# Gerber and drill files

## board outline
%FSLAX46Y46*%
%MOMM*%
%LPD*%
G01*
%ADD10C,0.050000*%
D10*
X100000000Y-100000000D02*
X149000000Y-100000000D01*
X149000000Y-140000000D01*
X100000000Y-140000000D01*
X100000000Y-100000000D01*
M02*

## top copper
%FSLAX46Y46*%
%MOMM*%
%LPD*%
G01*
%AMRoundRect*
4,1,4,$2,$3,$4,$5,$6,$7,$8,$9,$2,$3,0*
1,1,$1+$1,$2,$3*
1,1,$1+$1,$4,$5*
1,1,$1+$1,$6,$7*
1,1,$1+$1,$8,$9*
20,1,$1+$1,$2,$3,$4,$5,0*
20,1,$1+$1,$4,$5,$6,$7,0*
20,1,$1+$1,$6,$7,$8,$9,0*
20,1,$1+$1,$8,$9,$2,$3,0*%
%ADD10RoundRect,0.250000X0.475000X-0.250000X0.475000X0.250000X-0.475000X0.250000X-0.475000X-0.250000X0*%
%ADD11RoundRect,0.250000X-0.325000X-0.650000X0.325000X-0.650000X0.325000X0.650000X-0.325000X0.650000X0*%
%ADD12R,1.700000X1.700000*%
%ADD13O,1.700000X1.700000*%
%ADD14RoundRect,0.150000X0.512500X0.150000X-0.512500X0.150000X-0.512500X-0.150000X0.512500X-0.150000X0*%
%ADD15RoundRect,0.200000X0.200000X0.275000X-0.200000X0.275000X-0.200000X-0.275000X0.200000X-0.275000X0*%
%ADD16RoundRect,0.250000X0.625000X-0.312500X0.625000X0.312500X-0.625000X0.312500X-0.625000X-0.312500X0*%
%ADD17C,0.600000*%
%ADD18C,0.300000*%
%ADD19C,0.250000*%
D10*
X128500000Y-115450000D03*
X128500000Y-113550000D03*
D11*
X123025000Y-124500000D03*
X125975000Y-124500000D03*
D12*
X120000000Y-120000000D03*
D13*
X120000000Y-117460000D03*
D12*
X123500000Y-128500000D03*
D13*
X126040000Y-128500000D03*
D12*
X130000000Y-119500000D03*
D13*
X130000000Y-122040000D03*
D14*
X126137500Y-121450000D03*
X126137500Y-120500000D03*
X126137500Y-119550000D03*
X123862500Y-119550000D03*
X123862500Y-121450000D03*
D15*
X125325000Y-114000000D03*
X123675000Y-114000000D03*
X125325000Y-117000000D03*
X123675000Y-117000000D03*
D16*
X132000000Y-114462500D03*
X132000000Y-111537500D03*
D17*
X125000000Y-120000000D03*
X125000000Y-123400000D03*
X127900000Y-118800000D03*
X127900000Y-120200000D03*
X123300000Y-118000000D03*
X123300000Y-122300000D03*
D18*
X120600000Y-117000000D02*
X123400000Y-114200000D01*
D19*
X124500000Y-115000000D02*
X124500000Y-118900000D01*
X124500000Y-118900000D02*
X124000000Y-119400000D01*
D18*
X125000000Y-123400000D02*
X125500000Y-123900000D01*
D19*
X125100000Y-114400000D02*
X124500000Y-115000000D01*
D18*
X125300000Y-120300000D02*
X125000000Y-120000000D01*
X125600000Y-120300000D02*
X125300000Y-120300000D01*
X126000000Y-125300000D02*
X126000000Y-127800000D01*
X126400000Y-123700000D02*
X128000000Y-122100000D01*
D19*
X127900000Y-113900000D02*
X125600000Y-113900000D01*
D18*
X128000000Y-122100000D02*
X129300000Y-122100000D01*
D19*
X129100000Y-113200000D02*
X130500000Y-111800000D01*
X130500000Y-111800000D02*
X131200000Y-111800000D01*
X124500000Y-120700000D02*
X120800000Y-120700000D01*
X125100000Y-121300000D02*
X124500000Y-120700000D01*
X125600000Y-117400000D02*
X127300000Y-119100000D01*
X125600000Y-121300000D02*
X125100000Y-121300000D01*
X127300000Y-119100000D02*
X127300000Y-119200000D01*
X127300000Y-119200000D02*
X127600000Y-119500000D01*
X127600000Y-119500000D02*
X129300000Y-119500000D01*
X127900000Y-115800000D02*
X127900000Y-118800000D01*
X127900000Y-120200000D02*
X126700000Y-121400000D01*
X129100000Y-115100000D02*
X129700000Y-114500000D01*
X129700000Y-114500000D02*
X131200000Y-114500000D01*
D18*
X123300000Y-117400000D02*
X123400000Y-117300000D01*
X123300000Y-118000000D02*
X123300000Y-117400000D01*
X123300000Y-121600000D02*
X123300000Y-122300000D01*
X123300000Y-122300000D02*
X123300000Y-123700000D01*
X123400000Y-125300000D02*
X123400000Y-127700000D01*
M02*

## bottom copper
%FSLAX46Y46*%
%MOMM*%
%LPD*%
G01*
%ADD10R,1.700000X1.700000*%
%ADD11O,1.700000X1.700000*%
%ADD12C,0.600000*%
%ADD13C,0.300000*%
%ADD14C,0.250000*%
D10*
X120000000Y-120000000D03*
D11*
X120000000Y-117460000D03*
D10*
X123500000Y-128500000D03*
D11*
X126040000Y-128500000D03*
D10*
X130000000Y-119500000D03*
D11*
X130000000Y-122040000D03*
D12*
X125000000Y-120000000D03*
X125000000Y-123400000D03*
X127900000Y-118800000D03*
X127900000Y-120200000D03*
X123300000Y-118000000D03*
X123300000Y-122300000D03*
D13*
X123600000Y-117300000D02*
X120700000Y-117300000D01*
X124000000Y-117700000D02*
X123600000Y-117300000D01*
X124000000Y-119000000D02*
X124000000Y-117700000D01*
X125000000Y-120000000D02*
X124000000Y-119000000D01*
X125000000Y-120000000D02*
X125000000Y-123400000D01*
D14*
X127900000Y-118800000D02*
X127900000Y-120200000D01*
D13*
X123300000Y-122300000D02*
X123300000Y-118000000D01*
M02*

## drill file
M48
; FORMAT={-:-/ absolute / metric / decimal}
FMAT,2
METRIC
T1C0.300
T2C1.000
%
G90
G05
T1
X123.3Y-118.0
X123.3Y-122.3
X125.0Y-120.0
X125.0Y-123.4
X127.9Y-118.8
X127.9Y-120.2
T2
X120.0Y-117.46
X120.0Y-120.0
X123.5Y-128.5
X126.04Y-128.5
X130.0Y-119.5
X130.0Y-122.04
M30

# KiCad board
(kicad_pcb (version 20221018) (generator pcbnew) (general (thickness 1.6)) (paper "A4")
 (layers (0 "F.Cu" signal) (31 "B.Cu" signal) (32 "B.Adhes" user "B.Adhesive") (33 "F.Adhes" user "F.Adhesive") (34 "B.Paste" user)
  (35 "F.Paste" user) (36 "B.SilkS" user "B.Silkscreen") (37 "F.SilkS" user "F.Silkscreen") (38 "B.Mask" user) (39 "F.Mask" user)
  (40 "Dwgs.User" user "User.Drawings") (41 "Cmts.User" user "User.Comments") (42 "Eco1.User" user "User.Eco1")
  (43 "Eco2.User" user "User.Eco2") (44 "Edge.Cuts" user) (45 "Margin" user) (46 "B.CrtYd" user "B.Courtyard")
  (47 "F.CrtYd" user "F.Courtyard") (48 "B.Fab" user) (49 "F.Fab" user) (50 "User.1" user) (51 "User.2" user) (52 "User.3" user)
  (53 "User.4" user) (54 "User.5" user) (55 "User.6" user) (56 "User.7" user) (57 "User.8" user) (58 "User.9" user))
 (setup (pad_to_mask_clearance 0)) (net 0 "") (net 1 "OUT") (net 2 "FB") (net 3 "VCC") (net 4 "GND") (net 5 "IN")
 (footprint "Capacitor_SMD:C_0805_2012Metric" (layer "F.Cu") (at 128.5 114.5 90)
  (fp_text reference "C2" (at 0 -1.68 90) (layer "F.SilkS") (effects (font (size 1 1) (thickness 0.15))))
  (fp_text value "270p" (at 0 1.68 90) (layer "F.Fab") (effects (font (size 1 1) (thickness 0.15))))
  (pad "1" smd roundrect (at -0.95 0 90) (size 1 1.45) (layers "F.Cu" "F.Paste" "F.Mask") (roundrect_rratio 0.25) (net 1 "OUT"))
  (pad "2" smd roundrect (at 0.95 0 90) (size 1 1.45) (layers "F.Cu" "F.Paste" "F.Mask") (roundrect_rratio 0.25) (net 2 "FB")))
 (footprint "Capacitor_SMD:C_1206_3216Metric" (layer "F.Cu") (at 124.5 124.5)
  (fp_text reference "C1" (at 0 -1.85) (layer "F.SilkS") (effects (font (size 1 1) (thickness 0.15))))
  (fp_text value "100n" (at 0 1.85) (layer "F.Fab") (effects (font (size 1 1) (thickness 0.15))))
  (pad "1" smd roundrect (at -1.475 0) (size 1.15 1.8) (layers "F.Cu" "F.Paste" "F.Mask") (roundrect_rratio 0.217391) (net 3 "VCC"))
  (pad "2" smd roundrect (at 1.475 0) (size 1.15 1.8) (layers "F.Cu" "F.Paste" "F.Mask") (roundrect_rratio 0.217391) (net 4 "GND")))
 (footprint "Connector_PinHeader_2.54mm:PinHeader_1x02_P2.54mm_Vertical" (layer "F.Cu") (at 120 120 180)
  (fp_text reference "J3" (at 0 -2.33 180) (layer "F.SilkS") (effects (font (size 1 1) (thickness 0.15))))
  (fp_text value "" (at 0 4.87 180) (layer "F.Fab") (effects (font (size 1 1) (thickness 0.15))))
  (pad "1" thru_hole rect (at 0 0 180) (size 1.7 1.7) (drill 1) (layers "*.Cu" "*.Mask") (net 1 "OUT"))
  (pad "2" thru_hole oval (at 0 2.54 180) (size 1.7 1.7) (drill 1) (layers "*.Cu" "*.Mask") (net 4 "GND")))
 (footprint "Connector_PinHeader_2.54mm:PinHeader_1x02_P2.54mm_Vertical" (layer "F.Cu") (at 123.5 128.5 90)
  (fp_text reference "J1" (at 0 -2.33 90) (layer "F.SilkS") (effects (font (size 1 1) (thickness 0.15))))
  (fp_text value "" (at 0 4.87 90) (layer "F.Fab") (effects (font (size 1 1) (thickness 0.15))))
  (pad "1" thru_hole rect (at 0 0 90) (size 1.7 1.7) (drill 1) (layers "*.Cu" "*.Mask") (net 3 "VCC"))
  (pad "2" thru_hole oval (at 0 2.54 90) (size 1.7 1.7) (drill 1) (layers "*.Cu" "*.Mask") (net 4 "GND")))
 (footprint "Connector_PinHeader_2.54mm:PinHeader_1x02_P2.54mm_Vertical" (layer "F.Cu") (at 130 119.5)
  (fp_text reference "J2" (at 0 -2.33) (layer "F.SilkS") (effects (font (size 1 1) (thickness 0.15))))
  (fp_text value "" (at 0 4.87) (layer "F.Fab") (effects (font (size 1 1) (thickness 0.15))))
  (pad "1" thru_hole rect (at 0 0) (size 1.7 1.7) (drill 1) (layers "*.Cu" "*.Mask") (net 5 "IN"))
  (pad "2" thru_hole oval (at 0 2.54) (size 1.7 1.7) (drill 1) (layers "*.Cu" "*.Mask") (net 4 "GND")))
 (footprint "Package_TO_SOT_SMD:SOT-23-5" (layer "F.Cu") (at 125 120.5 180)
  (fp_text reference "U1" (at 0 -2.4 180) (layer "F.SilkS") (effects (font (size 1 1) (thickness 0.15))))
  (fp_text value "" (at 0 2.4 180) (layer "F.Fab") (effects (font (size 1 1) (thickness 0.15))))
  (pad "1" smd roundrect (at -1.1375 -0.95 180) (size 1.325 0.6) (layers "F.Cu" "F.Paste" "F.Mask") (roundrect_rratio 0.25) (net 1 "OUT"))
  (pad "2" smd roundrect (at -1.1375 0 180) (size 1.325 0.6) (layers "F.Cu" "F.Paste" "F.Mask") (roundrect_rratio 0.25) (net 4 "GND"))
  (pad "3" smd roundrect (at -1.1375 0.95 180) (size 1.325 0.6) (layers "F.Cu" "F.Paste" "F.Mask") (roundrect_rratio 0.25))
  (pad "4" smd roundrect (at 1.1375 0.95 180) (size 1.325 0.6) (layers "F.Cu" "F.Paste" "F.Mask") (roundrect_rratio 0.25) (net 2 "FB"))
  (pad "5" smd roundrect (at 1.1375 -0.95 180) (size 1.325 0.6) (layers "F.Cu" "F.Paste" "F.Mask") (roundrect_rratio 0.25) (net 3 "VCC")))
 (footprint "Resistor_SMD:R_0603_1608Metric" (layer "F.Cu") (at 124.5 114 180)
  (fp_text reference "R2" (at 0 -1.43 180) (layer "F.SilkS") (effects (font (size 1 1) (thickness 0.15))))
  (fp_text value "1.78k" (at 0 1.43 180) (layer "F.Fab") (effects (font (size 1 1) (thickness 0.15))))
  (pad "1" smd roundrect (at -0.825 0 180) (size 0.8 0.95) (layers "F.Cu" "F.Paste" "F.Mask") (roundrect_rratio 0.25) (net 2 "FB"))
  (pad "2" smd roundrect (at 0.825 0 180) (size 0.8 0.95) (layers "F.Cu" "F.Paste" "F.Mask") (roundrect_rratio 0.25) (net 4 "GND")))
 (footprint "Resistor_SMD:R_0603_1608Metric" (layer "F.Cu") (at 124.5 117 180)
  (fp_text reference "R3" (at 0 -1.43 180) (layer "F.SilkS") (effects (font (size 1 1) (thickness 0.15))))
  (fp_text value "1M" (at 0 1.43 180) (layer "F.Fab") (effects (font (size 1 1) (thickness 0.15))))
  (pad "1" smd roundrect (at -0.825 0 180) (size 0.8 0.95) (layers "F.Cu" "F.Paste" "F.Mask") (roundrect_rratio 0.25) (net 5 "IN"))
  (pad "2" smd roundrect (at 0.825 0 180) (size 0.8 0.95) (layers "F.Cu" "F.Paste" "F.Mask") (roundrect_rratio 0.25) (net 3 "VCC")))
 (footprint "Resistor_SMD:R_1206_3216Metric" (layer "F.Cu") (at 132 113 90)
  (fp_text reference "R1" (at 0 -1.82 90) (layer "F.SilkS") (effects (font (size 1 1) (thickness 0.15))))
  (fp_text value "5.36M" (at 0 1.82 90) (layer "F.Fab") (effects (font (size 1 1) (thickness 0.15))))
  (pad "1" smd roundrect (at -1.4625 0 90) (size 1.125 1.75) (layers "F.Cu" "F.Paste" "F.Mask") (roundrect_rratio 0.222222) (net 1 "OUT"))
  (pad "2" smd roundrect (at 1.4625 0 90) (size 1.125 1.75) (layers "F.Cu" "F.Paste" "F.Mask") (roundrect_rratio 0.222222) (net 2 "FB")))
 (gr_rect (start 100 100) (end 149 140) (stroke (width 0.05) (type default)) (fill none) (layer "Edge.Cuts"))
 (segment (start 120.6 117) (end 123.4 114.2) (width 0.3) (layer "F.Cu") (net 4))
 (segment (start 124.5 115) (end 124.5 118.9) (width 0.25) (layer "F.Cu") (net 2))
 (segment (start 124.5 118.9) (end 124 119.4) (width 0.25) (layer "F.Cu") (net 2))
 (segment (start 125 123.4) (end 125.5 123.9) (width 0.3) (layer "F.Cu") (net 4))
 (segment (start 125.1 114.4) (end 124.5 115) (width 0.25) (layer "F.Cu") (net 2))
 (segment (start 125.3 120.3) (end 125 120) (width 0.3) (layer "F.Cu") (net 4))
 (segment (start 125.6 120.3) (end 125.3 120.3) (width 0.3) (layer "F.Cu") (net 4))
 (segment (start 126 125.3) (end 126 127.8) (width 0.3) (layer "F.Cu") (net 4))
 (segment (start 126.4 123.7) (end 128 122.1) (width 0.3) (layer "F.Cu") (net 4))
 (segment (start 127.9 113.9) (end 125.6 113.9) (width 0.25) (layer "F.Cu") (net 2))
 (segment (start 128 122.1) (end 129.3 122.1) (width 0.3) (layer "F.Cu") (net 4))
 (segment (start 129.1 113.2) (end 130.5 111.8) (width 0.25) (layer "F.Cu") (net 2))
 (segment (start 130.5 111.8) (end 131.2 111.8) (width 0.25) (layer "F.Cu") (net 2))
 (via (at 125 120) (size 0.6) (drill 0.3) (layers "F.Cu" "B.Cu") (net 4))
 (via (at 125 123.4) (size 0.6) (drill 0.3) (layers "F.Cu" "B.Cu") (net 4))
 (segment (start 123.6 117.3) (end 120.7 117.3) (width 0.3) (layer "B.Cu") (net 4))
 (segment (start 124 117.7) (end 123.6 117.3) (width 0.3) (layer "B.Cu") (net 4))
 (segment (start 124 119) (end 124 117.7) (width 0.3) (layer "B.Cu") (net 4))
 (segment (start 124.5 120.7) (end 120.8 120.7) (width 0.25) (layer "F.Cu") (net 1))
 (segment (start 125 120) (end 124 119) (width 0.3) (layer "B.Cu") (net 4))
 (segment (start 125 120) (end 125 123.4) (width 0.3) (layer "B.Cu") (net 4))
 (segment (start 125.1 121.3) (end 124.5 120.7) (width 0.25) (layer "F.Cu") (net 1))
 (segment (start 125.6 117.4) (end 127.3 119.1) (width 0.25) (layer "F.Cu") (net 5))
 (segment (start 125.6 121.3) (end 125.1 121.3) (width 0.25) (layer "F.Cu") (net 1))
 (segment (start 127.3 119.1) (end 127.3 119.2) (width 0.25) (layer "F.Cu") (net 5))
 (segment (start 127.3 119.2) (end 127.6 119.5) (width 0.25) (layer "F.Cu") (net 5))
 (segment (start 127.6 119.5) (end 129.3 119.5) (width 0.25) (layer "F.Cu") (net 5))
 (segment (start 127.9 115.8) (end 127.9 118.8) (width 0.25) (layer "F.Cu") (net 1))
 (segment (start 127.9 120.2) (end 126.7 121.4) (width 0.25) (layer "F.Cu") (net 1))
 (segment (start 129.1 115.1) (end 129.7 114.5) (width 0.25) (layer "F.Cu") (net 1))
 (segment (start 129.7 114.5) (end 131.2 114.5) (width 0.25) (layer "F.Cu") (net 1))
 (via (at 127.9 118.8) (size 0.6) (drill 0.3) (layers "F.Cu" "B.Cu") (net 1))
 (via (at 127.9 120.2) (size 0.6) (drill 0.3) (layers "F.Cu" "B.Cu") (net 1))
 (segment (start 123.3 117.4) (end 123.4 117.3) (width 0.3) (layer "F.Cu") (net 3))
 (segment (start 123.3 118) (end 123.3 117.4) (width 0.3) (layer "F.Cu") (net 3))
 (segment (start 123.3 121.6) (end 123.3 122.3) (width 0.3) (layer "F.Cu") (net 3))
 (segment (start 123.3 122.3) (end 123.3 123.7) (width 0.3) (layer "F.Cu") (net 3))
 (segment (start 123.4 125.3) (end 123.4 127.7) (width 0.3) (layer "F.Cu") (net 3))
 (segment (start 127.9 118.8) (end 127.9 120.2) (width 0.25) (layer "B.Cu") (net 1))
 (via (at 123.3 118) (size 0.6) (drill 0.3) (layers "F.Cu" "B.Cu") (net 3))
 (via (at 123.3 122.3) (size 0.6) (drill 0.3) (layers "F.Cu" "B.Cu") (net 3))
 (segment (start 123.3 122.3) (end 123.3 118) (width 0.3) (layer "B.Cu") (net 3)))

